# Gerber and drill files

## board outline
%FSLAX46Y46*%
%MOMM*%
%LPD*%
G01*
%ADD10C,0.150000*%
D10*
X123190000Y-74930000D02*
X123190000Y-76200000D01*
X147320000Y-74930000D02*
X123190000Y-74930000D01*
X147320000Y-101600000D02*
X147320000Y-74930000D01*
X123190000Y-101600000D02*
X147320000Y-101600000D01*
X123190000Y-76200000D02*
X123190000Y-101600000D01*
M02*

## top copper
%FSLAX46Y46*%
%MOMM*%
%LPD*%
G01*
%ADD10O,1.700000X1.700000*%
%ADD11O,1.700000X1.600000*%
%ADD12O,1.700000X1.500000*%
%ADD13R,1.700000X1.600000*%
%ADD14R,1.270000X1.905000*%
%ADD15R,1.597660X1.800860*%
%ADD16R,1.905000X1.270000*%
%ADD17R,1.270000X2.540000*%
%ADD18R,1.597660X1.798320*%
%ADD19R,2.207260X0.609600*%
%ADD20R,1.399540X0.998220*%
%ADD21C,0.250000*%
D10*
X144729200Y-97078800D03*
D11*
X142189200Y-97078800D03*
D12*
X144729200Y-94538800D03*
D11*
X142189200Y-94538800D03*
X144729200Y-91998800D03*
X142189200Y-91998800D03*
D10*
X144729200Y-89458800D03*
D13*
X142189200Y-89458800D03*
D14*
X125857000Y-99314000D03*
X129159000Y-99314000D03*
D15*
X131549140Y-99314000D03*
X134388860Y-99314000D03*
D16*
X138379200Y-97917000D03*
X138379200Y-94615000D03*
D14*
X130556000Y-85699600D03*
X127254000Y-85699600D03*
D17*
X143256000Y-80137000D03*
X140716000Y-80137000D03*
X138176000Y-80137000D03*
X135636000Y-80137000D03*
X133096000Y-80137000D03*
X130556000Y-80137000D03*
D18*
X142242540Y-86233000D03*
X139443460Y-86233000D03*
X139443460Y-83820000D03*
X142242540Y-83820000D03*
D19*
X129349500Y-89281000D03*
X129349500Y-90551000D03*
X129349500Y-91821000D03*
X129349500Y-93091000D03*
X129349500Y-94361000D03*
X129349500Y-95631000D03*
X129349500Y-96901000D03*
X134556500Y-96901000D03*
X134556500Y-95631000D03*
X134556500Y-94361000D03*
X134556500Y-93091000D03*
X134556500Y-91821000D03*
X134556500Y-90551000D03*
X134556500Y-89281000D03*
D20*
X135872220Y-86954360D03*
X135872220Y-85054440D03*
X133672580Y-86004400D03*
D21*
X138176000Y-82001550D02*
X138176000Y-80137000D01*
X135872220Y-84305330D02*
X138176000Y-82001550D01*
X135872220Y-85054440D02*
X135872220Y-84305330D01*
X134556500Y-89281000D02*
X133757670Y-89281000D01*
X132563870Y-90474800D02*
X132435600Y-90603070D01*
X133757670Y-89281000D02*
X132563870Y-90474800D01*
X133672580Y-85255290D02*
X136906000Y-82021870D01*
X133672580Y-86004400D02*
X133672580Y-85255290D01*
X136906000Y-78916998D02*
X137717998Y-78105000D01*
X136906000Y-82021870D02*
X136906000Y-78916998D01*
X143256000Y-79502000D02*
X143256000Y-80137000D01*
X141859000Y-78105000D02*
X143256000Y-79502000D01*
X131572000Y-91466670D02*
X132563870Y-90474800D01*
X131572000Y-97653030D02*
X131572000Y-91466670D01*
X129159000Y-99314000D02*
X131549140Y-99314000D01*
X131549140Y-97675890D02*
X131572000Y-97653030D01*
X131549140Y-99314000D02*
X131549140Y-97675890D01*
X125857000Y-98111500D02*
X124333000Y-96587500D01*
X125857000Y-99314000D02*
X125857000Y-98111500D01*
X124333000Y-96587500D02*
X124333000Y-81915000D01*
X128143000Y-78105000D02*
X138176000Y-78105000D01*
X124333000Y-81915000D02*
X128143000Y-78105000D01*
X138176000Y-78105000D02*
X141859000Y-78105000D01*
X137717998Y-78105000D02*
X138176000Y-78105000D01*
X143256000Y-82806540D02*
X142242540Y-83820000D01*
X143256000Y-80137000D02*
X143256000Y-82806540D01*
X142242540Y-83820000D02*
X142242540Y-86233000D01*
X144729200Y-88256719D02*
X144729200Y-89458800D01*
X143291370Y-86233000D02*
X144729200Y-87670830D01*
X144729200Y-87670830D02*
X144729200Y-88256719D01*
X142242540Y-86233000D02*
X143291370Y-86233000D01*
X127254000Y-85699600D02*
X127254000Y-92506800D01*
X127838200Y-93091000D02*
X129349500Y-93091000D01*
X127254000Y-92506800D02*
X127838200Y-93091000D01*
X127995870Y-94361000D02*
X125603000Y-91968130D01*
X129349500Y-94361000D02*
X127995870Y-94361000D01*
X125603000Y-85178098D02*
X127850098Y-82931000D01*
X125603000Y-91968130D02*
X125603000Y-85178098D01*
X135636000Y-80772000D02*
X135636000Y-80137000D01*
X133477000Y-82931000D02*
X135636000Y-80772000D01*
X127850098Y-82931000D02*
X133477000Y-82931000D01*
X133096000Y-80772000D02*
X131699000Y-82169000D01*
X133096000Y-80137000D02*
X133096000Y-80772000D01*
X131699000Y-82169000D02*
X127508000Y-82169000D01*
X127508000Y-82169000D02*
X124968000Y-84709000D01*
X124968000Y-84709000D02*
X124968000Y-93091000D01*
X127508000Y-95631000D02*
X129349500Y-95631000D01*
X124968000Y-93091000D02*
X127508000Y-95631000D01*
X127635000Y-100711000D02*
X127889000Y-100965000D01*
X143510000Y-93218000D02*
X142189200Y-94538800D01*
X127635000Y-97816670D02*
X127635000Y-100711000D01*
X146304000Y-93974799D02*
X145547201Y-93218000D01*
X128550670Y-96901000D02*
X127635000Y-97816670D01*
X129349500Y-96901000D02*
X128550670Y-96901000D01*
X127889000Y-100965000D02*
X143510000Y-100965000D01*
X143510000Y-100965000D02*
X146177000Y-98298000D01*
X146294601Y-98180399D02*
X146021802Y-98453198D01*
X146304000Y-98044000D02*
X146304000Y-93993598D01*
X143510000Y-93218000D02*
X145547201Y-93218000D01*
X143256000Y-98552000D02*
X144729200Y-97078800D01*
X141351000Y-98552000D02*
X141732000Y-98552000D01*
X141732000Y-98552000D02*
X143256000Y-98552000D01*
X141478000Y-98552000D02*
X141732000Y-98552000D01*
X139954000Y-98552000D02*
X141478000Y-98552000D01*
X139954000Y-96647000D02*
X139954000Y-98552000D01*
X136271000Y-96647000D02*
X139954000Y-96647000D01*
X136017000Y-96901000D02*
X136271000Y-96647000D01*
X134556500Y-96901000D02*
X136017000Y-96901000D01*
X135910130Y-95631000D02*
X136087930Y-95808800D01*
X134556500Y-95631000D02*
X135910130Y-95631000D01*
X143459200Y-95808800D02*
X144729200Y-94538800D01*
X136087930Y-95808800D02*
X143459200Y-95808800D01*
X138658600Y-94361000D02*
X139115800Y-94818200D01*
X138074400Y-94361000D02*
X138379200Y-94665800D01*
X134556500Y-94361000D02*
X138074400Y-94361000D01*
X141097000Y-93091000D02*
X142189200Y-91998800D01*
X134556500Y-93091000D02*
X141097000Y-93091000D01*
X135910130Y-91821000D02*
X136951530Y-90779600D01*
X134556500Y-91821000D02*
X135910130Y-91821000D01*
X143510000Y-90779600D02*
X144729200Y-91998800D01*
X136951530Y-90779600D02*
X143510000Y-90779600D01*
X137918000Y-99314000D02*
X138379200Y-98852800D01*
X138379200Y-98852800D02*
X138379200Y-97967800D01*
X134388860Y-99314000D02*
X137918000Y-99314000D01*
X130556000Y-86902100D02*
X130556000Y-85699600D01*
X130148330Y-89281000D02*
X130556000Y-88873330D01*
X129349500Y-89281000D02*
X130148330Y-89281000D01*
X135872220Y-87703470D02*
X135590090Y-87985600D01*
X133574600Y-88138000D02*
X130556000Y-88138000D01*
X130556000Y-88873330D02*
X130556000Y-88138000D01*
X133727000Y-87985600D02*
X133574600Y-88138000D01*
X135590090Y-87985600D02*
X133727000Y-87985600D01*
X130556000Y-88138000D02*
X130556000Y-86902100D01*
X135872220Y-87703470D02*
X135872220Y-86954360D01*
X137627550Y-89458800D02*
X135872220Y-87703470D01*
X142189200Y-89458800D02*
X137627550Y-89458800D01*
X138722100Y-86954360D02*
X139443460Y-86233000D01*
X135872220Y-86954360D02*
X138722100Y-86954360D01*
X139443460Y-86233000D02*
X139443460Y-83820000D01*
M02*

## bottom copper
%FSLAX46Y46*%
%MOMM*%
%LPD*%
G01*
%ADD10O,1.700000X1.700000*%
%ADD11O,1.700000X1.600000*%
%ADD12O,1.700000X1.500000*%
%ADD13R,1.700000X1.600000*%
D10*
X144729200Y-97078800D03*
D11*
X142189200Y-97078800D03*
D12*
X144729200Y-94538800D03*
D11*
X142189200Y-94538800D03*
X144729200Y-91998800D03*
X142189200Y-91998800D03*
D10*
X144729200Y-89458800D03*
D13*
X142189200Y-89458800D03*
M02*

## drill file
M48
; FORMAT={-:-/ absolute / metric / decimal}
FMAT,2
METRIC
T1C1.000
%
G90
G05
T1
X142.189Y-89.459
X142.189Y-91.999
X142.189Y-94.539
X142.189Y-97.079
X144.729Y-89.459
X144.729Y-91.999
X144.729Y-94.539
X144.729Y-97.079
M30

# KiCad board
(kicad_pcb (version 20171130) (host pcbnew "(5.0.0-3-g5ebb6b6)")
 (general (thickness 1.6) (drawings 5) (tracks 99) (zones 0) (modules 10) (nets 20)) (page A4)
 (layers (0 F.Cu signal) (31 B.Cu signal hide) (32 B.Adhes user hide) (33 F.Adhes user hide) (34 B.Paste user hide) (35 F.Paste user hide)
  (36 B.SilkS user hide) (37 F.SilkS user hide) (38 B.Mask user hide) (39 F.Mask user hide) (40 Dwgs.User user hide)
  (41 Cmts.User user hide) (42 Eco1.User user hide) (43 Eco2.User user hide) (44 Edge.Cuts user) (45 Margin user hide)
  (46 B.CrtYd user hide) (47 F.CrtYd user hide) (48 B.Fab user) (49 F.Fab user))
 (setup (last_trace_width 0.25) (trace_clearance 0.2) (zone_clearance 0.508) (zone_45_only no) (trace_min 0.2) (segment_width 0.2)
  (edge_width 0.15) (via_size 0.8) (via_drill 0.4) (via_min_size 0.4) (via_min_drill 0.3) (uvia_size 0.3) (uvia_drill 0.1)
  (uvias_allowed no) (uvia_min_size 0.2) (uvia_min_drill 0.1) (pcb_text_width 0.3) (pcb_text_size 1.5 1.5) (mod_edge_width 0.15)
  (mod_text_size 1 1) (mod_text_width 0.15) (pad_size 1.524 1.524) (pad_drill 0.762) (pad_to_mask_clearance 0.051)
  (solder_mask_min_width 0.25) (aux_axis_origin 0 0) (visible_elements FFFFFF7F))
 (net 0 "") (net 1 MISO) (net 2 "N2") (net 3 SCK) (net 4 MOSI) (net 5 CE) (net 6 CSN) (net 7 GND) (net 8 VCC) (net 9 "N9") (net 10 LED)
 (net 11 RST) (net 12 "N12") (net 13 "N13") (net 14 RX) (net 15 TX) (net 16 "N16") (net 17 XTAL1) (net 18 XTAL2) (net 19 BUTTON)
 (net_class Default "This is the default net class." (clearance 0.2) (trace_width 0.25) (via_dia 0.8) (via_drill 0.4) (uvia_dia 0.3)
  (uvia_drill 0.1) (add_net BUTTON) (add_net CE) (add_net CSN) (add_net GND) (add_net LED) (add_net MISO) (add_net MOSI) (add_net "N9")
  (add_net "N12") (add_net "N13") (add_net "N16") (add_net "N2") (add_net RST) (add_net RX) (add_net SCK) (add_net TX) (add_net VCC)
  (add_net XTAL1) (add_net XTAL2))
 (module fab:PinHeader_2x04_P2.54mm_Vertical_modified (layer F.Cu) (at 142.1892 89.4588)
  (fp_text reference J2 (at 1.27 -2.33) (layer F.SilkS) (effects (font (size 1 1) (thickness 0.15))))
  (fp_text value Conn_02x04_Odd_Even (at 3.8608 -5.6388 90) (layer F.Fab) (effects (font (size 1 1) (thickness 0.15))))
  (pad 8 thru_hole oval (at 2.54 7.62) (size 1.7 1.7) (drill 1) (layers *.Cu *.Mask) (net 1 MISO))
  (pad 7 thru_hole oval (at 0 7.62) (size 1.7 1.6) (drill 1) (layers *.Cu *.Mask) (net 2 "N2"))
  (pad 6 thru_hole oval (at 2.54 5.08) (size 1.7 1.5) (drill 1) (layers *.Cu *.Mask) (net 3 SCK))
  (pad 5 thru_hole oval (at 0 5.08) (size 1.7 1.6) (drill 1) (layers *.Cu *.Mask) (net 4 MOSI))
  (pad 4 thru_hole oval (at 2.54 2.54) (size 1.7 1.6) (drill 1) (layers *.Cu *.Mask) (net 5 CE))
  (pad 3 thru_hole oval (at 0 2.54) (size 1.7 1.6) (drill 1) (layers *.Cu *.Mask) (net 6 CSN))
  (pad 2 thru_hole oval (at 2.54 0) (size 1.7 1.7) (drill 1) (layers *.Cu *.Mask) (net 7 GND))
  (pad 1 thru_hole rect (at 0 0) (size 1.7 1.6) (drill 1) (layers *.Cu *.Mask) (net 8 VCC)))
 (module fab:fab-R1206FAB (layer F.Cu) (at 127.508 99.314)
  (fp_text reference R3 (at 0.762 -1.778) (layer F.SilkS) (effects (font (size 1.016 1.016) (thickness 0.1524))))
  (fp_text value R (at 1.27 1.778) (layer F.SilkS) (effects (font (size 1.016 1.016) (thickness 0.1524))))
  (pad 1 smd rect (at -1.651 0) (size 1.27 1.905) (layers F.Cu F.Paste F.Mask) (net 7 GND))
  (pad 2 smd rect (at 1.651 0) (size 1.27 1.905) (layers F.Cu F.Paste F.Mask) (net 7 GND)))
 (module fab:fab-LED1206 (layer F.Cu) (at 132.969 99.314)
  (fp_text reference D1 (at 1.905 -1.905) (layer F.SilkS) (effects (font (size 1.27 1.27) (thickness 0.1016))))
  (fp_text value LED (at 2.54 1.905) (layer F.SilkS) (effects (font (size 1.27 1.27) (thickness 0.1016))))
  (pad 1 smd rect (at -1.41986 0) (size 1.59766 1.80086) (layers F.Cu F.Paste F.Mask) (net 7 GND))
  (pad 2 smd rect (at 1.41986 0) (size 1.59766 1.80086) (layers F.Cu F.Paste F.Mask) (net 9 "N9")))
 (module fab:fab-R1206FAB (layer F.Cu) (at 138.3792 96.266 270)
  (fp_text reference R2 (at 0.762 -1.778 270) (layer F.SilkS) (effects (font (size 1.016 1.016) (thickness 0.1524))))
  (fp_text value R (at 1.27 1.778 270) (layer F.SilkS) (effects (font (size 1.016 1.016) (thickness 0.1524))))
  (pad 2 smd rect (at 1.651 0 270) (size 1.27 1.905) (layers F.Cu F.Paste F.Mask) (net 9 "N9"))
  (pad 1 smd rect (at -1.651 0 270) (size 1.27 1.905) (layers F.Cu F.Paste F.Mask) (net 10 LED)))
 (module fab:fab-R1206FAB (layer F.Cu) (at 128.905 85.6996 180)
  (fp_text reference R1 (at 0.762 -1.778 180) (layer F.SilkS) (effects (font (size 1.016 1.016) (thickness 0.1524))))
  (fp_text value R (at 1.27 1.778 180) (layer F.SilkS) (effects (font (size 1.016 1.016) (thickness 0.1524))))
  (pad 1 smd rect (at -1.651 0 180) (size 1.27 1.905) (layers F.Cu F.Paste F.Mask) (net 8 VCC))
  (pad 2 smd rect (at 1.651 0 180) (size 1.27 1.905) (layers F.Cu F.Paste F.Mask) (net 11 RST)))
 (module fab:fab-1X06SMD (layer F.Cu) (at 136.906 80.137 270)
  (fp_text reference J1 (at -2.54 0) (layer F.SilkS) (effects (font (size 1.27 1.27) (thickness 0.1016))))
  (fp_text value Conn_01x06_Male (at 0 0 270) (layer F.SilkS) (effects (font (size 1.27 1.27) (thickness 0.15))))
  (pad 1 smd rect (at 0 -6.35 270) (size 2.54 1.27) (layers F.Cu F.Paste F.Mask) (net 7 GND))
  (pad 2 smd rect (at 0 -3.81 270) (size 2.54 1.27) (layers F.Cu F.Paste F.Mask) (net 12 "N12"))
  (pad 3 smd rect (at 0 -1.27 270) (size 2.54 1.27) (layers F.Cu F.Paste F.Mask) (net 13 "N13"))
  (pad 4 smd rect (at 0 1.27 270) (size 2.54 1.27) (layers F.Cu F.Paste F.Mask) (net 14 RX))
  (pad 5 smd rect (at 0 3.81 270) (size 2.54 1.27) (layers F.Cu F.Paste F.Mask) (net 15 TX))
  (pad 6 smd rect (at 0 6.35 270) (size 2.54 1.27) (layers F.Cu F.Paste F.Mask) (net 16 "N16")))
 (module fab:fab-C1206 (layer F.Cu) (at 140.843 86.233)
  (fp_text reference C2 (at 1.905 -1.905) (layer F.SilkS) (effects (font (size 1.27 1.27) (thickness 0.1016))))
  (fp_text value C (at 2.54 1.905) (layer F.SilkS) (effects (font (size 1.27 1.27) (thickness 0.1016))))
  (pad 2 smd rect (at 1.39954 0) (size 1.59766 1.79832) (layers F.Cu F.Paste F.Mask) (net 7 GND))
  (pad 1 smd rect (at -1.39954 0) (size 1.59766 1.79832) (layers F.Cu F.Paste F.Mask) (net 8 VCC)))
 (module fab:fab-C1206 (layer F.Cu) (at 140.843 83.82)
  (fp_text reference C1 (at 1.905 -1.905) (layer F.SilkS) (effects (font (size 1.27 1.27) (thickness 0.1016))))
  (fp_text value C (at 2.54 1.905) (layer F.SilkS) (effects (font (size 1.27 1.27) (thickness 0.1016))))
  (pad 1 smd rect (at -1.39954 0) (size 1.59766 1.79832) (layers F.Cu F.Paste F.Mask) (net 8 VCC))
  (pad 2 smd rect (at 1.39954 0) (size 1.59766 1.79832) (layers F.Cu F.Paste F.Mask) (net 7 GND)))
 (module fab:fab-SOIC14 (layer F.Cu) (at 131.953 93.091 270)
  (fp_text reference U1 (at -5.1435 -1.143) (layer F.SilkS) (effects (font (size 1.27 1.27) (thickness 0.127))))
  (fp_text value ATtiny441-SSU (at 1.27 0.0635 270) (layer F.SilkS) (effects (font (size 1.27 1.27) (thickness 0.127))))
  (pad 1 smd rect (at -3.81 2.6035 270) (size 0.6096 2.20726) (layers F.Cu F.Paste F.Mask) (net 8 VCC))
  (pad 2 smd rect (at -2.54 2.6035 270) (size 0.6096 2.20726) (layers F.Cu F.Paste F.Mask) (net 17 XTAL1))
  (pad 3 smd rect (at -1.27 2.6035 270) (size 0.6096 2.20726) (layers F.Cu F.Paste F.Mask) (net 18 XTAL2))
  (pad 4 smd rect (at 0 2.6035 270) (size 0.6096 2.20726) (layers F.Cu F.Paste F.Mask) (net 11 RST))
  (pad 5 smd rect (at 1.27 2.6035 270) (size 0.6096 2.20726) (layers F.Cu F.Paste F.Mask) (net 14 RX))
  (pad 6 smd rect (at 2.54 2.6035 270) (size 0.6096 2.20726) (layers F.Cu F.Paste F.Mask) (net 15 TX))
  (pad 7 smd rect (at 3.81 2.6035 270) (size 0.6096 2.20726) (layers F.Cu F.Paste F.Mask) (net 4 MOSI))
  (pad 8 smd rect (at 3.81 -2.6035 270) (size 0.6096 2.20726) (layers F.Cu F.Paste F.Mask) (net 1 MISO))
  (pad 9 smd rect (at 2.54 -2.6035 270) (size 0.6096 2.20726) (layers F.Cu F.Paste F.Mask) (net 3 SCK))
  (pad 10 smd rect (at 1.27 -2.6035 270) (size 0.6096 2.20726) (layers F.Cu F.Paste F.Mask) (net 10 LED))
  (pad 11 smd rect (at 0 -2.6035 270) (size 0.6096 2.20726) (layers F.Cu F.Paste F.Mask) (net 6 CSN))
  (pad 12 smd rect (at -1.27 -2.6035 270) (size 0.6096 2.20726) (layers F.Cu F.Paste F.Mask) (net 5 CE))
  (pad 13 smd rect (at -2.54 -2.6035 270) (size 0.6096 2.20726) (layers F.Cu F.Paste F.Mask) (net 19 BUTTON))
  (pad 14 smd rect (at -3.81 -2.6035 270) (size 0.6096 2.20726) (layers F.Cu F.Paste F.Mask) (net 7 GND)))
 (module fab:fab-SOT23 (layer F.Cu) (at 134.7724 86.0044 90)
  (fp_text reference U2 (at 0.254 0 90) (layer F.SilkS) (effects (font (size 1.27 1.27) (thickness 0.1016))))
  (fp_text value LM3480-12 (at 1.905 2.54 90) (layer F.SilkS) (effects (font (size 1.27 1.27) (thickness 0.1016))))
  (pad 1 smd rect (at -0.94996 1.09982 90) (size 0.99822 1.39954) (layers F.Cu F.Paste F.Mask) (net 8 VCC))
  (pad 2 smd rect (at 0.94996 1.09982 90) (size 0.99822 1.39954) (layers F.Cu F.Paste F.Mask) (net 13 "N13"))
  (pad 3 smd rect (at 0 -1.09982 90) (size 0.99822 1.39954) (layers F.Cu F.Paste F.Mask) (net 7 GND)))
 (gr_line (start 123.19 74.93) (end 123.19 76.2) (layer Edge.Cuts) (width 0.15))
 (gr_line (start 147.32 74.93) (end 123.19 74.93) (layer Edge.Cuts) (width 0.15))
 (gr_line (start 147.32 101.6) (end 147.32 74.93) (layer Edge.Cuts) (width 0.15))
 (gr_line (start 123.19 101.6) (end 147.32 101.6) (layer Edge.Cuts) (width 0.15))
 (gr_line (start 123.19 76.2) (end 123.19 101.6) (layer Edge.Cuts) (width 0.15))
 (segment (start 138.176 82.00155) (end 138.176 80.137) (width 0.25) (layer F.Cu) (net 13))
 (segment (start 135.87222 84.30533) (end 138.176 82.00155) (width 0.25) (layer F.Cu) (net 13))
 (segment (start 135.87222 85.05444) (end 135.87222 84.30533) (width 0.25) (layer F.Cu) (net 13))
 (segment (start 134.5565 89.281) (end 133.75767 89.281) (width 0.25) (layer F.Cu) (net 7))
 (segment (start 132.56387 90.4748) (end 132.4356 90.60307) (width 0.25) (layer F.Cu) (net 7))
 (segment (start 133.75767 89.281) (end 132.56387 90.4748) (width 0.25) (layer F.Cu) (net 7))
 (segment (start 133.67258 85.25529) (end 136.906 82.02187) (width 0.25) (layer F.Cu) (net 7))
 (segment (start 133.67258 86.0044) (end 133.67258 85.25529) (width 0.25) (layer F.Cu) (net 7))
 (segment (start 136.906 78.916998) (end 137.717998 78.105) (width 0.25) (layer F.Cu) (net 7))
 (segment (start 136.906 82.02187) (end 136.906 78.916998) (width 0.25) (layer F.Cu) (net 7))
 (segment (start 143.256 79.502) (end 143.256 80.137) (width 0.25) (layer F.Cu) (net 7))
 (segment (start 141.859 78.105) (end 143.256 79.502) (width 0.25) (layer F.Cu) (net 7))
 (segment (start 131.572 91.46667) (end 132.56387 90.4748) (width 0.25) (layer F.Cu) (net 7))
 (segment (start 131.572 97.65303) (end 131.572 91.46667) (width 0.25) (layer F.Cu) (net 7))
 (segment (start 129.159 99.314) (end 131.54914 99.314) (width 0.25) (layer F.Cu) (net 7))
 (segment (start 131.54914 97.67589) (end 131.572 97.65303) (width 0.25) (layer F.Cu) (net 7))
 (segment (start 131.54914 99.314) (end 131.54914 97.67589) (width 0.25) (layer F.Cu) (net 7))
 (segment (start 125.857 98.1115) (end 124.333 96.5875) (width 0.25) (layer F.Cu) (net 7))
 (segment (start 125.857 99.314) (end 125.857 98.1115) (width 0.25) (layer F.Cu) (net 7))
 (segment (start 124.333 96.5875) (end 124.333 81.915) (width 0.25) (layer F.Cu) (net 7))
 (segment (start 128.143 78.105) (end 138.176 78.105) (width 0.25) (layer F.Cu) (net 7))
 (segment (start 124.333 81.915) (end 128.143 78.105) (width 0.25) (layer F.Cu) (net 7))
 (segment (start 138.176 78.105) (end 141.859 78.105) (width 0.25) (layer F.Cu) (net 7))
 (segment (start 137.717998 78.105) (end 138.176 78.105) (width 0.25) (layer F.Cu) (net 7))
 (segment (start 143.256 82.80654) (end 142.24254 83.82) (width 0.25) (layer F.Cu) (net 7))
 (segment (start 143.256 80.137) (end 143.256 82.80654) (width 0.25) (layer F.Cu) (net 7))
 (segment (start 142.24254 83.82) (end 142.24254 86.233) (width 0.25) (layer F.Cu) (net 7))
 (segment (start 144.7292 88.256719) (end 144.7292 89.4588) (width 0.25) (layer F.Cu) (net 7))
 (segment (start 143.29137 86.233) (end 144.7292 87.67083) (width 0.25) (layer F.Cu) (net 7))
 (segment (start 144.7292 87.67083) (end 144.7292 88.256719) (width 0.25) (layer F.Cu) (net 7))
 (segment (start 142.24254 86.233) (end 143.29137 86.233) (width 0.25) (layer F.Cu) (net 7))
 (segment (start 127.254 85.6996) (end 127.254 92.5068) (width 0.25) (layer F.Cu) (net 11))
 (segment (start 127.8382 93.091) (end 129.3495 93.091) (width 0.25) (layer F.Cu) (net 11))
 (segment (start 127.254 92.5068) (end 127.8382 93.091) (width 0.25) (layer F.Cu) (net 11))
 (segment (start 127.99587 94.361) (end 125.603 91.96813) (width 0.25) (layer F.Cu) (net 14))
 (segment (start 129.3495 94.361) (end 127.99587 94.361) (width 0.25) (layer F.Cu) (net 14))
 (segment (start 125.603 85.178098) (end 127.850098 82.931) (width 0.25) (layer F.Cu) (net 14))
 (segment (start 125.603 91.96813) (end 125.603 85.178098) (width 0.25) (layer F.Cu) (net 14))
 (segment (start 135.636 80.772) (end 135.636 80.137) (width 0.25) (layer F.Cu) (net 14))
 (segment (start 133.477 82.931) (end 135.636 80.772) (width 0.25) (layer F.Cu) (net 14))
 (segment (start 127.850098 82.931) (end 133.477 82.931) (width 0.25) (layer F.Cu) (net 14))
 (segment (start 133.096 80.772) (end 131.699 82.169) (width 0.25) (layer F.Cu) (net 15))
 (segment (start 133.096 80.137) (end 133.096 80.772) (width 0.25) (layer F.Cu) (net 15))
 (segment (start 131.699 82.169) (end 127.508 82.169) (width 0.25) (layer F.Cu) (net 15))
 (segment (start 127.508 82.169) (end 124.968 84.709) (width 0.25) (layer F.Cu) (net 15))
 (segment (start 124.968 84.709) (end 124.968 93.091) (width 0.25) (layer F.Cu) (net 15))
 (segment (start 127.508 95.631) (end 129.3495 95.631) (width 0.25) (layer F.Cu) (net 15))
 (segment (start 124.968 93.091) (end 127.508 95.631) (width 0.25) (layer F.Cu) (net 15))
 (segment (start 127.635 100.711) (end 127.889 100.965) (width 0.25) (layer F.Cu) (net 4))
 (segment (start 143.51 93.218) (end 142.1892 94.5388) (width 0.25) (layer F.Cu) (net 4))
 (segment (start 127.635 97.81667) (end 127.635 100.711) (width 0.25) (layer F.Cu) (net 4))
 (segment (start 146.304 93.974799) (end 145.547201 93.218) (width 0.25) (layer F.Cu) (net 4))
 (segment (start 128.55067 96.901) (end 127.635 97.81667) (width 0.25) (layer F.Cu) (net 4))
 (segment (start 129.3495 96.901) (end 128.55067 96.901) (width 0.25) (layer F.Cu) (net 4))
 (segment (start 127.889 100.965) (end 143.51 100.965) (width 0.25) (layer F.Cu) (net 4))
 (segment (start 143.51 100.965) (end 146.177 98.298) (width 0.25) (layer F.Cu) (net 4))
 (segment (start 146.294601 98.180399) (end 146.021802 98.453198) (width 0.25) (layer F.Cu) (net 4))
 (segment (start 146.304 98.044) (end 146.304 93.993598) (width 0.25) (layer F.Cu) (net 4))
 (segment (start 143.51 93.218) (end 145.547201 93.218) (width 0.25) (layer F.Cu) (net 4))
 (segment (start 143.256 98.552) (end 144.7292 97.0788) (width 0.25) (layer F.Cu) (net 1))
 (segment (start 141.351 98.552) (end 141.732 98.552) (width 0.25) (layer F.Cu) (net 1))
 (segment (start 141.732 98.552) (end 143.256 98.552) (width 0.25) (layer F.Cu) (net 1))
 (segment (start 141.478 98.552) (end 141.732 98.552) (width 0.25) (layer F.Cu) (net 1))
 (segment (start 139.954 98.552) (end 141.478 98.552) (width 0.25) (layer F.Cu) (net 1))
 (segment (start 139.954 96.647) (end 139.954 98.552) (width 0.25) (layer F.Cu) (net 1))
 (segment (start 136.271 96.647) (end 139.954 96.647) (width 0.25) (layer F.Cu) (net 1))
 (segment (start 136.017 96.901) (end 136.271 96.647) (width 0.25) (layer F.Cu) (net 1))
 (segment (start 134.5565 96.901) (end 136.017 96.901) (width 0.25) (layer F.Cu) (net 1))
 (segment (start 135.91013 95.631) (end 136.08793 95.8088) (width 0.25) (layer F.Cu) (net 3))
 (segment (start 134.5565 95.631) (end 135.91013 95.631) (width 0.25) (layer F.Cu) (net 3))
 (segment (start 143.4592 95.8088) (end 144.7292 94.5388) (width 0.25) (layer F.Cu) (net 3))
 (segment (start 136.08793 95.8088) (end 143.4592 95.8088) (width 0.25) (layer F.Cu) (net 3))
 (segment (start 138.6586 94.361) (end 139.1158 94.8182) (width 0.25) (layer F.Cu) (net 10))
 (segment (start 138.0744 94.361) (end 138.3792 94.6658) (width 0.25) (layer F.Cu) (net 10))
 (segment (start 134.5565 94.361) (end 138.0744 94.361) (width 0.25) (layer F.Cu) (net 10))
 (segment (start 141.097 93.091) (end 142.1892 91.9988) (width 0.25) (layer F.Cu) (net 6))
 (segment (start 134.5565 93.091) (end 141.097 93.091) (width 0.25) (layer F.Cu) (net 6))
 (segment (start 135.91013 91.821) (end 136.95153 90.7796) (width 0.25) (layer F.Cu) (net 5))
 (segment (start 134.5565 91.821) (end 135.91013 91.821) (width 0.25) (layer F.Cu) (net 5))
 (segment (start 143.51 90.7796) (end 144.7292 91.9988) (width 0.25) (layer F.Cu) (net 5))
 (segment (start 136.95153 90.7796) (end 143.51 90.7796) (width 0.25) (layer F.Cu) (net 5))
 (segment (start 137.918 99.314) (end 138.3792 98.8528) (width 0.25) (layer F.Cu) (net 9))
 (segment (start 138.3792 98.8528) (end 138.3792 97.9678) (width 0.25) (layer F.Cu) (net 9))
 (segment (start 134.38886 99.314) (end 137.918 99.314) (width 0.25) (layer F.Cu) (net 9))
 (segment (start 130.556 86.9021) (end 130.556 85.6996) (width 0.25) (layer F.Cu) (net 8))
 (segment (start 130.14833 89.281) (end 130.556 88.87333) (width 0.25) (layer F.Cu) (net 8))
 (segment (start 129.3495 89.281) (end 130.14833 89.281) (width 0.25) (layer F.Cu) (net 8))
 (segment (start 135.87222 87.70347) (end 135.59009 87.9856) (width 0.25) (layer F.Cu) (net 8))
 (segment (start 133.5746 88.138) (end 130.556 88.138) (width 0.25) (layer F.Cu) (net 8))
 (segment (start 130.556 88.87333) (end 130.556 88.138) (width 0.25) (layer F.Cu) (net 8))
 (segment (start 133.727 87.9856) (end 133.5746 88.138) (width 0.25) (layer F.Cu) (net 8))
 (segment (start 135.59009 87.9856) (end 133.727 87.9856) (width 0.25) (layer F.Cu) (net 8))
 (segment (start 130.556 88.138) (end 130.556 86.9021) (width 0.25) (layer F.Cu) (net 8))
 (segment (start 135.87222 87.70347) (end 135.87222 86.95436) (width 0.25) (layer F.Cu) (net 8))
 (segment (start 137.62755 89.4588) (end 135.87222 87.70347) (width 0.25) (layer F.Cu) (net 8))
 (segment (start 142.1892 89.4588) (end 137.62755 89.4588) (width 0.25) (layer F.Cu) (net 8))
 (segment (start 138.7221 86.95436) (end 139.44346 86.233) (width 0.25) (layer F.Cu) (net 8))
 (segment (start 135.87222 86.95436) (end 138.7221 86.95436) (width 0.25) (layer F.Cu) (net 8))
 (segment (start 139.44346 86.233) (end 139.44346 83.82) (width 0.25) (layer F.Cu) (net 8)))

